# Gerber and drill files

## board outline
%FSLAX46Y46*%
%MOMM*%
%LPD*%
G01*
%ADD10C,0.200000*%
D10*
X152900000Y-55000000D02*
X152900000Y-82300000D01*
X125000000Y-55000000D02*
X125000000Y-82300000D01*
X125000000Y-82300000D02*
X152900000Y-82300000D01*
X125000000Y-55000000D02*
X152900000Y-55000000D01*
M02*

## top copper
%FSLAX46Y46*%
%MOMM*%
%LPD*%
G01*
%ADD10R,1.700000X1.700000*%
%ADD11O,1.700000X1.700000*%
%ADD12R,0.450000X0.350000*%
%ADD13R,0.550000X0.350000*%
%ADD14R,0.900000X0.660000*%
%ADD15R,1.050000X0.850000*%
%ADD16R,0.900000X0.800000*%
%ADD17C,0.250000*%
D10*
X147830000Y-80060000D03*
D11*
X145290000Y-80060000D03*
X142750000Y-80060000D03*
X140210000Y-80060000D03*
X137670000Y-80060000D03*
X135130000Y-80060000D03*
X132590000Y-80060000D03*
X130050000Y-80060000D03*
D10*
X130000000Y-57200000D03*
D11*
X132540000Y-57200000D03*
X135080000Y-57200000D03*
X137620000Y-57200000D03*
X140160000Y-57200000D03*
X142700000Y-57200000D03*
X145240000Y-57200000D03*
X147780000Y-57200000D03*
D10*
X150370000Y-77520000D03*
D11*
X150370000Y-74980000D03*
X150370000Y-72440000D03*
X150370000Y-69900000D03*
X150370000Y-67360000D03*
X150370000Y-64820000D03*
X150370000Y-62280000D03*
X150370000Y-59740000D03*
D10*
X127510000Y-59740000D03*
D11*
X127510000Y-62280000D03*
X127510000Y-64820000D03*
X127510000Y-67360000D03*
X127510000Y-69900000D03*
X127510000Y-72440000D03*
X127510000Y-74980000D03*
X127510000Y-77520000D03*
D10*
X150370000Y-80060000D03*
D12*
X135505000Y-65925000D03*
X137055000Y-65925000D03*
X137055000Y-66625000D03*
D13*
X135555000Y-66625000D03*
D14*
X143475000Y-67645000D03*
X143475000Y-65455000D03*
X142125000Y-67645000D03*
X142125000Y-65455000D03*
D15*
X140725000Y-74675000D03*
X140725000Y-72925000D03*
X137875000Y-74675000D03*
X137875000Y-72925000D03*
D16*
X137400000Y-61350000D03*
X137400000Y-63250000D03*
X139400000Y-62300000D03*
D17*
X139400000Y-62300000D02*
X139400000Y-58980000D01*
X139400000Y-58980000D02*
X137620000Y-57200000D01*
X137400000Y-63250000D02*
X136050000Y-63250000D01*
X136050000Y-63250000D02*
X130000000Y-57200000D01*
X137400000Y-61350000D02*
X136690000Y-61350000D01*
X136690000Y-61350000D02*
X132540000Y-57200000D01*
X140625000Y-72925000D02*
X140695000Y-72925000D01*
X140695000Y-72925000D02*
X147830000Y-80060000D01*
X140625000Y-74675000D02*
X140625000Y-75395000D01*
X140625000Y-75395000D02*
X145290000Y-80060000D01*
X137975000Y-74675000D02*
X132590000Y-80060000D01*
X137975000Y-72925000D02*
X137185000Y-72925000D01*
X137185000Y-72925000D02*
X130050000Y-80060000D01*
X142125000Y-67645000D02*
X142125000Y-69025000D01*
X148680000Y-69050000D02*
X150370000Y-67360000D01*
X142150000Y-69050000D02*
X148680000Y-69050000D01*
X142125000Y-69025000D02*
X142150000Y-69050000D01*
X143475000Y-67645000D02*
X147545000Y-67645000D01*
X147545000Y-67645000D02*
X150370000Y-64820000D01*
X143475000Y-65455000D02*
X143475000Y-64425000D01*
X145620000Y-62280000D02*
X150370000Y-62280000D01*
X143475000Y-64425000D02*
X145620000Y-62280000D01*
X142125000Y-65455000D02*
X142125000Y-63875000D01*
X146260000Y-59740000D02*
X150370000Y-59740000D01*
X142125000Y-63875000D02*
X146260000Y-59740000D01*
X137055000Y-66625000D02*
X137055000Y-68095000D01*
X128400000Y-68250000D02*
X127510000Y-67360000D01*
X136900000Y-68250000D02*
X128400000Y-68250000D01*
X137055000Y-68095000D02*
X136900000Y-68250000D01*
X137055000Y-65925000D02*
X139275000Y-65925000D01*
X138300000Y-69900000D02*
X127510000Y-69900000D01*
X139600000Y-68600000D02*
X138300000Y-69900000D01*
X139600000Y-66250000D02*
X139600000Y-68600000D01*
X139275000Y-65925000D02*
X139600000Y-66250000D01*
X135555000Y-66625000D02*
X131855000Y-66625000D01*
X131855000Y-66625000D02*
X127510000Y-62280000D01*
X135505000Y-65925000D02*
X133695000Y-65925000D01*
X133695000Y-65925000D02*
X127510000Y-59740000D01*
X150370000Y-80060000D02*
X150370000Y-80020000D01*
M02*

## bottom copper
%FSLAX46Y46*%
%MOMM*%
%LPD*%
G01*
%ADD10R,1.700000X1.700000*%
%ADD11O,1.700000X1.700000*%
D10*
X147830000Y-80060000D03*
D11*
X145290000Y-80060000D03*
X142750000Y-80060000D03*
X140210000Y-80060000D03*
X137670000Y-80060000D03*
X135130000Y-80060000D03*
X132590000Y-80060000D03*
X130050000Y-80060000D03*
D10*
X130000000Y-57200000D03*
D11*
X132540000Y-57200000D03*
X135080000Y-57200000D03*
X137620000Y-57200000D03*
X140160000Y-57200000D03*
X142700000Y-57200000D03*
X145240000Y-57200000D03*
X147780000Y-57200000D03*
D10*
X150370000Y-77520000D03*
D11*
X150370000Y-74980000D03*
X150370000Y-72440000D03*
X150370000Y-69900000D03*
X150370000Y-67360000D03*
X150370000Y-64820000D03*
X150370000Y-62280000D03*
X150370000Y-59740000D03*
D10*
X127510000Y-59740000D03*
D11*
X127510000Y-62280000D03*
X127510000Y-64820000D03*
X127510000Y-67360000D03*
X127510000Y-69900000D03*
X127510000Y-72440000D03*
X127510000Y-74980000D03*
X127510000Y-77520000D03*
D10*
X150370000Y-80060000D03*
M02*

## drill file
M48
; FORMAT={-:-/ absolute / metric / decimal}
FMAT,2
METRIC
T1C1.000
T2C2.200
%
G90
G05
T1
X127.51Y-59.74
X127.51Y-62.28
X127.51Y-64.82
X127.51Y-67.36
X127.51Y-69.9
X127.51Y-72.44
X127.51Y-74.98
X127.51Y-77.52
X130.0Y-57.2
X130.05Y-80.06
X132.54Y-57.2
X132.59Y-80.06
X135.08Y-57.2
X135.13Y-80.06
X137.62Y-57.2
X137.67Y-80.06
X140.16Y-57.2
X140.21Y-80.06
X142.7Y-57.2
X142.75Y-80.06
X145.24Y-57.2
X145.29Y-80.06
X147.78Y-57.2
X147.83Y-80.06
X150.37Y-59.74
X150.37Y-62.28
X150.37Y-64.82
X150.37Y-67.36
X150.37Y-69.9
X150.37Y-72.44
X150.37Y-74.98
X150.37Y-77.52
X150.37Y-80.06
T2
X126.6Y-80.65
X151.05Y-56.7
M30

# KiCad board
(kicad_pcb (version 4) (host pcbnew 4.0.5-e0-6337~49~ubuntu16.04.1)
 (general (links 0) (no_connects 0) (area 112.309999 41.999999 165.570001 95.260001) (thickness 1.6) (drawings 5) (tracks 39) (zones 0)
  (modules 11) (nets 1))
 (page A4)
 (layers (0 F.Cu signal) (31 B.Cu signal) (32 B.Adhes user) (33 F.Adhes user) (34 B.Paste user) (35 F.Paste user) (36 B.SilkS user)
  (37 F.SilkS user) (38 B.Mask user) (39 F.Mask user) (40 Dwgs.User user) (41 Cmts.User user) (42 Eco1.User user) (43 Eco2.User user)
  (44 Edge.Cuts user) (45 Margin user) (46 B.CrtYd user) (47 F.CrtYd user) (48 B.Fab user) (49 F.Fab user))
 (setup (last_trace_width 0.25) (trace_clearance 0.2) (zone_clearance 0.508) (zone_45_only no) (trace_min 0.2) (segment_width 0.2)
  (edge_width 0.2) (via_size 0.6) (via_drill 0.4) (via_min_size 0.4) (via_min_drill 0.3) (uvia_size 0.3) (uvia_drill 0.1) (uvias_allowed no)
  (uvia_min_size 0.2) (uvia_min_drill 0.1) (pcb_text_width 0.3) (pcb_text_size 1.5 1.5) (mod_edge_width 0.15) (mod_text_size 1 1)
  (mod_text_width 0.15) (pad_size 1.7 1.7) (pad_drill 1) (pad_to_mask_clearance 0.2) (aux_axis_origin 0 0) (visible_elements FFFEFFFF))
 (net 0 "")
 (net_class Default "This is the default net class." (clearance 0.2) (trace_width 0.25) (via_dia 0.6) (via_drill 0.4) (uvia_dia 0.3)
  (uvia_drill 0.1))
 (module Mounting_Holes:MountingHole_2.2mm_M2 (layer F.Cu) (at 151.05 56.7)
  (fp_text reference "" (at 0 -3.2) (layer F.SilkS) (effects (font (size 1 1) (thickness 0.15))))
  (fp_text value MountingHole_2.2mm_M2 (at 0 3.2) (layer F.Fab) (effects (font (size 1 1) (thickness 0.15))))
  (pad 1 np_thru_hole circle (at 0 0) (size 2.2 2.2) (drill 2.2) (layers *.Cu *.Mask)))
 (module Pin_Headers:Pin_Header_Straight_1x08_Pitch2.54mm (layer F.Cu) (at 147.83 80.06 270)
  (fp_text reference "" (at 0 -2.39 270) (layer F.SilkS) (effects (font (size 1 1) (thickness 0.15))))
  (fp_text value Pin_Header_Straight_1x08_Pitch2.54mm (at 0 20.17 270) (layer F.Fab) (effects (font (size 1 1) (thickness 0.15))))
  (pad 1 thru_hole rect (at 0 0 270) (size 1.7 1.7) (drill 1) (layers *.Cu *.Mask))
  (pad 2 thru_hole oval (at 0 2.54 270) (size 1.7 1.7) (drill 1) (layers *.Cu *.Mask))
  (pad 3 thru_hole oval (at 0 5.08 270) (size 1.7 1.7) (drill 1) (layers *.Cu *.Mask))
  (pad 4 thru_hole oval (at 0 7.62 270) (size 1.7 1.7) (drill 1) (layers *.Cu *.Mask))
  (pad 5 thru_hole oval (at 0 10.16 270) (size 1.7 1.7) (drill 1) (layers *.Cu *.Mask))
  (pad 6 thru_hole oval (at 0 12.7 270) (size 1.7 1.7) (drill 1) (layers *.Cu *.Mask))
  (pad 7 thru_hole oval (at 0 15.24 270) (size 1.7 1.7) (drill 1) (layers *.Cu *.Mask))
  (pad 8 thru_hole oval (at 0 17.78 270) (size 1.7 1.7) (drill 1) (layers *.Cu *.Mask)))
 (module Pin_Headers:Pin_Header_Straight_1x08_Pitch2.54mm (layer F.Cu) (at 130 57.2 90)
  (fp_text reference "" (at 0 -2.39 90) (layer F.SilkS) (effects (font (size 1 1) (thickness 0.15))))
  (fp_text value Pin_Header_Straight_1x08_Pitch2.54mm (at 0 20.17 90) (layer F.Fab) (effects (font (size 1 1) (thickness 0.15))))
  (pad 1 thru_hole rect (at 0 0 90) (size 1.7 1.7) (drill 1) (layers *.Cu *.Mask))
  (pad 2 thru_hole oval (at 0 2.54 90) (size 1.7 1.7) (drill 1) (layers *.Cu *.Mask))
  (pad 3 thru_hole oval (at 0 5.08 90) (size 1.7 1.7) (drill 1) (layers *.Cu *.Mask))
  (pad 4 thru_hole oval (at 0 7.62 90) (size 1.7 1.7) (drill 1) (layers *.Cu *.Mask))
  (pad 5 thru_hole oval (at 0 10.16 90) (size 1.7 1.7) (drill 1) (layers *.Cu *.Mask))
  (pad 6 thru_hole oval (at 0 12.7 90) (size 1.7 1.7) (drill 1) (layers *.Cu *.Mask))
  (pad 7 thru_hole oval (at 0 15.24 90) (size 1.7 1.7) (drill 1) (layers *.Cu *.Mask))
  (pad 8 thru_hole oval (at 0 17.78 90) (size 1.7 1.7) (drill 1) (layers *.Cu *.Mask)))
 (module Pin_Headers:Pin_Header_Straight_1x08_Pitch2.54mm (layer F.Cu) (at 150.37 77.52 180)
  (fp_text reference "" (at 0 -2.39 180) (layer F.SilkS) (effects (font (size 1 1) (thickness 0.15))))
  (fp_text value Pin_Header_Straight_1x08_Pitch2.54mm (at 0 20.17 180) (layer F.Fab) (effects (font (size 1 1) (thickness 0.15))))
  (pad 1 thru_hole rect (at 0 0 180) (size 1.7 1.7) (drill 1) (layers *.Cu *.Mask))
  (pad 2 thru_hole oval (at 0 2.54 180) (size 1.7 1.7) (drill 1) (layers *.Cu *.Mask))
  (pad 3 thru_hole oval (at 0 5.08 180) (size 1.7 1.7) (drill 1) (layers *.Cu *.Mask))
  (pad 4 thru_hole oval (at 0 7.62 180) (size 1.7 1.7) (drill 1) (layers *.Cu *.Mask))
  (pad 5 thru_hole oval (at 0 10.16 180) (size 1.7 1.7) (drill 1) (layers *.Cu *.Mask))
  (pad 6 thru_hole oval (at 0 12.7 180) (size 1.7 1.7) (drill 1) (layers *.Cu *.Mask))
  (pad 7 thru_hole oval (at 0 15.24 180) (size 1.7 1.7) (drill 1) (layers *.Cu *.Mask))
  (pad 8 thru_hole oval (at 0 17.78 180) (size 1.7 1.7) (drill 1) (layers *.Cu *.Mask)))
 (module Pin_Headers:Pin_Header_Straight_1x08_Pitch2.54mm (layer F.Cu) (at 127.51 59.74)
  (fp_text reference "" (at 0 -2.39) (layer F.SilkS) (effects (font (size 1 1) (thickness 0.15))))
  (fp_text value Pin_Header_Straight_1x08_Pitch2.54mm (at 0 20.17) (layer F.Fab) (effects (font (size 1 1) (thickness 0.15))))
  (pad 1 thru_hole rect (at 0 0) (size 1.7 1.7) (drill 1) (layers *.Cu *.Mask))
  (pad 2 thru_hole oval (at 0 2.54) (size 1.7 1.7) (drill 1) (layers *.Cu *.Mask))
  (pad 3 thru_hole oval (at 0 5.08) (size 1.7 1.7) (drill 1) (layers *.Cu *.Mask))
  (pad 4 thru_hole oval (at 0 7.62) (size 1.7 1.7) (drill 1) (layers *.Cu *.Mask))
  (pad 5 thru_hole oval (at 0 10.16) (size 1.7 1.7) (drill 1) (layers *.Cu *.Mask))
  (pad 6 thru_hole oval (at 0 12.7) (size 1.7 1.7) (drill 1) (layers *.Cu *.Mask))
  (pad 7 thru_hole oval (at 0 15.24) (size 1.7 1.7) (drill 1) (layers *.Cu *.Mask))
  (pad 8 thru_hole oval (at 0 17.78) (size 1.7 1.7) (drill 1) (layers *.Cu *.Mask)))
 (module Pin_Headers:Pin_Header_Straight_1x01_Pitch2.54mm (layer F.Cu) (at 150.37 80.06)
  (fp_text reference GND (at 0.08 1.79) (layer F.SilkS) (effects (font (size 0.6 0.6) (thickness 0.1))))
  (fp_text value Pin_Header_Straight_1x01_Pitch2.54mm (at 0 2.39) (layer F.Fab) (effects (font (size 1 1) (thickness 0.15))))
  (pad 1 thru_hole rect (at 0 0) (size 1.7 1.7) (drill 1) (layers *.Cu *.Mask)))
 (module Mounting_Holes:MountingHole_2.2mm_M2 (layer F.Cu) (at 126.6 80.65)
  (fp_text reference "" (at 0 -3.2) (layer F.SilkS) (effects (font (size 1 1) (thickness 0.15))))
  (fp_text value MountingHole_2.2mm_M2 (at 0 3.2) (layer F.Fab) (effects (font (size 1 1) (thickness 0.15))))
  (pad 1 np_thru_hole circle (at 0 0) (size 2.2 2.2) (drill 2.2) (layers *.Cu *.Mask)))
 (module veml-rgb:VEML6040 (layer F.Cu) (at 136.45 65.2)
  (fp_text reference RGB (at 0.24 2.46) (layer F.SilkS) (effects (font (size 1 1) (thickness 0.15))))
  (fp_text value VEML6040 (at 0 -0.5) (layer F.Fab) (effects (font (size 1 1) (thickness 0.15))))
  (pad 1 smd rect (at -0.945 0.725) (size 0.45 0.35) (layers F.Cu F.Paste F.Mask))
  (pad 2 smd rect (at 0.605 0.725) (size 0.45 0.35) (layers F.Cu F.Paste F.Mask))
  (pad 3 smd rect (at 0.605 1.425) (size 0.45 0.35) (layers F.Cu F.Paste F.Mask))
  (pad 4 smd rect (at -0.895 1.425) (size 0.55 0.35) (layers F.Cu F.Paste F.Mask)))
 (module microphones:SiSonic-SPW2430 (layer F.Cu) (at 141.55 65)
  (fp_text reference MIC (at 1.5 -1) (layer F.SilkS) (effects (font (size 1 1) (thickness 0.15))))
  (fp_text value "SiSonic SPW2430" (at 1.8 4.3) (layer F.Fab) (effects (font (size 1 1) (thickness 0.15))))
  (pad +v smd rect (at 1.925 2.645) (size 0.9 0.66) (layers F.Cu F.Paste F.Mask))
  (pad +v smd rect (at 1.925 0.455) (size 0.9 0.66) (layers F.Cu F.Paste F.Mask))
  (pad GND smd rect (at 0.575 2.645) (size 0.9 0.66) (layers F.Cu F.Paste F.Mask))
  (pad +v smd rect (at 0.575 0.455) (size 0.9 0.66) (layers F.Cu F.Paste F.Mask)))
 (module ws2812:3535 (layer F.Cu) (at 139.3 73.8)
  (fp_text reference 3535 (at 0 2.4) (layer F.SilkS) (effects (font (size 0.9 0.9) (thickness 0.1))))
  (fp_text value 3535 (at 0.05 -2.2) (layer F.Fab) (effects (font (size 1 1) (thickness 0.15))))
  (pad IN smd rect (at 1.325 0.875) (size 1.05 0.85) (drill (offset 0.1 0)) (layers F.Cu F.Paste F.Mask))
  (pad VDD smd rect (at 1.325 -0.875) (size 1.05 0.85) (drill (offset 0.1 0)) (layers F.Cu F.Paste F.Mask))
  (pad GND smd rect (at -1.325 0.875) (size 1.05 0.85) (drill (offset -0.1 0)) (layers F.Cu F.Paste F.Mask))
  (pad OUT smd rect (at -1.325 -0.875) (size 1.05 0.85) (drill (offset -0.1 0)) (layers F.Cu F.Paste F.Mask)))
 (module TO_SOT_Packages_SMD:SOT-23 (layer F.Cu) (at 138.4 62.3)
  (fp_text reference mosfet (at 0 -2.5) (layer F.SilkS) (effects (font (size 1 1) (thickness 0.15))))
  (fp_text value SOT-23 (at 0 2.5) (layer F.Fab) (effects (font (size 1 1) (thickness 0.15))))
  (pad 1 smd rect (at -1 -0.95) (size 0.9 0.8) (layers F.Cu F.Paste F.Mask))
  (pad 2 smd rect (at -1 0.95) (size 0.9 0.8) (layers F.Cu F.Paste F.Mask))
  (pad 3 smd rect (at 1 0) (size 0.9 0.8) (layers F.Cu F.Paste F.Mask)))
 (gr_line (start 152.9 55) (end 152.9 82.3) (angle 90) (layer Edge.Cuts) (width 0.2))
 (gr_line (start 125 55) (end 125 82.3) (angle 90) (layer Edge.Cuts) (width 0.2))
 (gr_line (start 125 82.3) (end 152.9 82.3) (angle 90) (layer Edge.Cuts) (width 0.2))
 (gr_line (start 125 55) (end 152.9 55) (angle 90) (layer Edge.Cuts) (width 0.2))
 (segment (start 139.4 62.3) (end 139.4 58.98) (width 0.25) (layer F.Cu) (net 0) (status 400000))
 (segment (start 139.4 58.98) (end 137.62 57.2) (width 0.25) (layer F.Cu) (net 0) (status 800000))
 (segment (start 137.4 63.25) (end 136.05 63.25) (width 0.25) (layer F.Cu) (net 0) (status 400000))
 (segment (start 136.05 63.25) (end 130 57.2) (width 0.25) (layer F.Cu) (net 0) (status 800000))
 (segment (start 137.4 61.35) (end 136.69 61.35) (width 0.25) (layer F.Cu) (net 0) (status 400000))
 (segment (start 136.69 61.35) (end 132.54 57.2) (width 0.25) (layer F.Cu) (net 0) (status 800000))
 (segment (start 140.625 72.925) (end 140.695 72.925) (width 0.25) (layer F.Cu) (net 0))
 (segment (start 140.695 72.925) (end 147.83 80.06) (width 0.25) (layer F.Cu) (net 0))
 (segment (start 140.625 74.675) (end 140.625 75.395) (width 0.25) (layer F.Cu) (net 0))
 (segment (start 140.625 75.395) (end 145.29 80.06) (width 0.25) (layer F.Cu) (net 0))
 (segment (start 137.975 74.675) (end 132.59 80.06) (width 0.25) (layer F.Cu) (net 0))
 (segment (start 137.975 72.925) (end 137.185 72.925) (width 0.25) (layer F.Cu) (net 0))
 (segment (start 137.185 72.925) (end 130.05 80.06) (width 0.25) (layer F.Cu) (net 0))
 (segment (start 142.125 67.645) (end 142.125 69.025) (width 0.25) (layer F.Cu) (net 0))
 (segment (start 148.68 69.05) (end 150.37 67.36) (width 0.25) (layer F.Cu) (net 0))
 (segment (start 142.15 69.05) (end 148.68 69.05) (width 0.25) (layer F.Cu) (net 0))
 (segment (start 142.125 69.025) (end 142.15 69.05) (width 0.25) (layer F.Cu) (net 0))
 (segment (start 143.475 67.645) (end 147.545 67.645) (width 0.25) (layer F.Cu) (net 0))
 (segment (start 147.545 67.645) (end 150.37 64.82) (width 0.25) (layer F.Cu) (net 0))
 (segment (start 143.475 65.455) (end 143.475 64.425) (width 0.25) (layer F.Cu) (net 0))
 (segment (start 145.62 62.28) (end 150.37 62.28) (width 0.25) (layer F.Cu) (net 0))
 (segment (start 143.475 64.425) (end 145.62 62.28) (width 0.25) (layer F.Cu) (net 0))
 (segment (start 142.125 65.455) (end 142.125 63.875) (width 0.25) (layer F.Cu) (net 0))
 (segment (start 146.26 59.74) (end 150.37 59.74) (width 0.25) (layer F.Cu) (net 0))
 (segment (start 142.125 63.875) (end 146.26 59.74) (width 0.25) (layer F.Cu) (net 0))
 (segment (start 137.055 66.625) (end 137.055 68.095) (width 0.25) (layer F.Cu) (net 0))
 (segment (start 128.4 68.25) (end 127.51 67.36) (width 0.25) (layer F.Cu) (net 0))
 (segment (start 136.9 68.25) (end 128.4 68.25) (width 0.25) (layer F.Cu) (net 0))
 (segment (start 137.055 68.095) (end 136.9 68.25) (width 0.25) (layer F.Cu) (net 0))
 (segment (start 137.055 65.925) (end 139.275 65.925) (width 0.25) (layer F.Cu) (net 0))
 (segment (start 138.3 69.9) (end 127.51 69.9) (width 0.25) (layer F.Cu) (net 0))
 (segment (start 139.6 68.6) (end 138.3 69.9) (width 0.25) (layer F.Cu) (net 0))
 (segment (start 139.6 66.25) (end 139.6 68.6) (width 0.25) (layer F.Cu) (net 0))
 (segment (start 139.275 65.925) (end 139.6 66.25) (width 0.25) (layer F.Cu) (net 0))
 (segment (start 135.555 66.625) (end 131.855 66.625) (width 0.25) (layer F.Cu) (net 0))
 (segment (start 131.855 66.625) (end 127.51 62.28) (width 0.25) (layer F.Cu) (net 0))
 (segment (start 135.505 65.925) (end 133.695 65.925) (width 0.25) (layer F.Cu) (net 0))
 (segment (start 133.695 65.925) (end 127.51 59.74) (width 0.25) (layer F.Cu) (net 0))
 (segment (start 150.37 80.06) (end 150.37 80.02) (width 0.25) (layer F.Cu) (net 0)))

